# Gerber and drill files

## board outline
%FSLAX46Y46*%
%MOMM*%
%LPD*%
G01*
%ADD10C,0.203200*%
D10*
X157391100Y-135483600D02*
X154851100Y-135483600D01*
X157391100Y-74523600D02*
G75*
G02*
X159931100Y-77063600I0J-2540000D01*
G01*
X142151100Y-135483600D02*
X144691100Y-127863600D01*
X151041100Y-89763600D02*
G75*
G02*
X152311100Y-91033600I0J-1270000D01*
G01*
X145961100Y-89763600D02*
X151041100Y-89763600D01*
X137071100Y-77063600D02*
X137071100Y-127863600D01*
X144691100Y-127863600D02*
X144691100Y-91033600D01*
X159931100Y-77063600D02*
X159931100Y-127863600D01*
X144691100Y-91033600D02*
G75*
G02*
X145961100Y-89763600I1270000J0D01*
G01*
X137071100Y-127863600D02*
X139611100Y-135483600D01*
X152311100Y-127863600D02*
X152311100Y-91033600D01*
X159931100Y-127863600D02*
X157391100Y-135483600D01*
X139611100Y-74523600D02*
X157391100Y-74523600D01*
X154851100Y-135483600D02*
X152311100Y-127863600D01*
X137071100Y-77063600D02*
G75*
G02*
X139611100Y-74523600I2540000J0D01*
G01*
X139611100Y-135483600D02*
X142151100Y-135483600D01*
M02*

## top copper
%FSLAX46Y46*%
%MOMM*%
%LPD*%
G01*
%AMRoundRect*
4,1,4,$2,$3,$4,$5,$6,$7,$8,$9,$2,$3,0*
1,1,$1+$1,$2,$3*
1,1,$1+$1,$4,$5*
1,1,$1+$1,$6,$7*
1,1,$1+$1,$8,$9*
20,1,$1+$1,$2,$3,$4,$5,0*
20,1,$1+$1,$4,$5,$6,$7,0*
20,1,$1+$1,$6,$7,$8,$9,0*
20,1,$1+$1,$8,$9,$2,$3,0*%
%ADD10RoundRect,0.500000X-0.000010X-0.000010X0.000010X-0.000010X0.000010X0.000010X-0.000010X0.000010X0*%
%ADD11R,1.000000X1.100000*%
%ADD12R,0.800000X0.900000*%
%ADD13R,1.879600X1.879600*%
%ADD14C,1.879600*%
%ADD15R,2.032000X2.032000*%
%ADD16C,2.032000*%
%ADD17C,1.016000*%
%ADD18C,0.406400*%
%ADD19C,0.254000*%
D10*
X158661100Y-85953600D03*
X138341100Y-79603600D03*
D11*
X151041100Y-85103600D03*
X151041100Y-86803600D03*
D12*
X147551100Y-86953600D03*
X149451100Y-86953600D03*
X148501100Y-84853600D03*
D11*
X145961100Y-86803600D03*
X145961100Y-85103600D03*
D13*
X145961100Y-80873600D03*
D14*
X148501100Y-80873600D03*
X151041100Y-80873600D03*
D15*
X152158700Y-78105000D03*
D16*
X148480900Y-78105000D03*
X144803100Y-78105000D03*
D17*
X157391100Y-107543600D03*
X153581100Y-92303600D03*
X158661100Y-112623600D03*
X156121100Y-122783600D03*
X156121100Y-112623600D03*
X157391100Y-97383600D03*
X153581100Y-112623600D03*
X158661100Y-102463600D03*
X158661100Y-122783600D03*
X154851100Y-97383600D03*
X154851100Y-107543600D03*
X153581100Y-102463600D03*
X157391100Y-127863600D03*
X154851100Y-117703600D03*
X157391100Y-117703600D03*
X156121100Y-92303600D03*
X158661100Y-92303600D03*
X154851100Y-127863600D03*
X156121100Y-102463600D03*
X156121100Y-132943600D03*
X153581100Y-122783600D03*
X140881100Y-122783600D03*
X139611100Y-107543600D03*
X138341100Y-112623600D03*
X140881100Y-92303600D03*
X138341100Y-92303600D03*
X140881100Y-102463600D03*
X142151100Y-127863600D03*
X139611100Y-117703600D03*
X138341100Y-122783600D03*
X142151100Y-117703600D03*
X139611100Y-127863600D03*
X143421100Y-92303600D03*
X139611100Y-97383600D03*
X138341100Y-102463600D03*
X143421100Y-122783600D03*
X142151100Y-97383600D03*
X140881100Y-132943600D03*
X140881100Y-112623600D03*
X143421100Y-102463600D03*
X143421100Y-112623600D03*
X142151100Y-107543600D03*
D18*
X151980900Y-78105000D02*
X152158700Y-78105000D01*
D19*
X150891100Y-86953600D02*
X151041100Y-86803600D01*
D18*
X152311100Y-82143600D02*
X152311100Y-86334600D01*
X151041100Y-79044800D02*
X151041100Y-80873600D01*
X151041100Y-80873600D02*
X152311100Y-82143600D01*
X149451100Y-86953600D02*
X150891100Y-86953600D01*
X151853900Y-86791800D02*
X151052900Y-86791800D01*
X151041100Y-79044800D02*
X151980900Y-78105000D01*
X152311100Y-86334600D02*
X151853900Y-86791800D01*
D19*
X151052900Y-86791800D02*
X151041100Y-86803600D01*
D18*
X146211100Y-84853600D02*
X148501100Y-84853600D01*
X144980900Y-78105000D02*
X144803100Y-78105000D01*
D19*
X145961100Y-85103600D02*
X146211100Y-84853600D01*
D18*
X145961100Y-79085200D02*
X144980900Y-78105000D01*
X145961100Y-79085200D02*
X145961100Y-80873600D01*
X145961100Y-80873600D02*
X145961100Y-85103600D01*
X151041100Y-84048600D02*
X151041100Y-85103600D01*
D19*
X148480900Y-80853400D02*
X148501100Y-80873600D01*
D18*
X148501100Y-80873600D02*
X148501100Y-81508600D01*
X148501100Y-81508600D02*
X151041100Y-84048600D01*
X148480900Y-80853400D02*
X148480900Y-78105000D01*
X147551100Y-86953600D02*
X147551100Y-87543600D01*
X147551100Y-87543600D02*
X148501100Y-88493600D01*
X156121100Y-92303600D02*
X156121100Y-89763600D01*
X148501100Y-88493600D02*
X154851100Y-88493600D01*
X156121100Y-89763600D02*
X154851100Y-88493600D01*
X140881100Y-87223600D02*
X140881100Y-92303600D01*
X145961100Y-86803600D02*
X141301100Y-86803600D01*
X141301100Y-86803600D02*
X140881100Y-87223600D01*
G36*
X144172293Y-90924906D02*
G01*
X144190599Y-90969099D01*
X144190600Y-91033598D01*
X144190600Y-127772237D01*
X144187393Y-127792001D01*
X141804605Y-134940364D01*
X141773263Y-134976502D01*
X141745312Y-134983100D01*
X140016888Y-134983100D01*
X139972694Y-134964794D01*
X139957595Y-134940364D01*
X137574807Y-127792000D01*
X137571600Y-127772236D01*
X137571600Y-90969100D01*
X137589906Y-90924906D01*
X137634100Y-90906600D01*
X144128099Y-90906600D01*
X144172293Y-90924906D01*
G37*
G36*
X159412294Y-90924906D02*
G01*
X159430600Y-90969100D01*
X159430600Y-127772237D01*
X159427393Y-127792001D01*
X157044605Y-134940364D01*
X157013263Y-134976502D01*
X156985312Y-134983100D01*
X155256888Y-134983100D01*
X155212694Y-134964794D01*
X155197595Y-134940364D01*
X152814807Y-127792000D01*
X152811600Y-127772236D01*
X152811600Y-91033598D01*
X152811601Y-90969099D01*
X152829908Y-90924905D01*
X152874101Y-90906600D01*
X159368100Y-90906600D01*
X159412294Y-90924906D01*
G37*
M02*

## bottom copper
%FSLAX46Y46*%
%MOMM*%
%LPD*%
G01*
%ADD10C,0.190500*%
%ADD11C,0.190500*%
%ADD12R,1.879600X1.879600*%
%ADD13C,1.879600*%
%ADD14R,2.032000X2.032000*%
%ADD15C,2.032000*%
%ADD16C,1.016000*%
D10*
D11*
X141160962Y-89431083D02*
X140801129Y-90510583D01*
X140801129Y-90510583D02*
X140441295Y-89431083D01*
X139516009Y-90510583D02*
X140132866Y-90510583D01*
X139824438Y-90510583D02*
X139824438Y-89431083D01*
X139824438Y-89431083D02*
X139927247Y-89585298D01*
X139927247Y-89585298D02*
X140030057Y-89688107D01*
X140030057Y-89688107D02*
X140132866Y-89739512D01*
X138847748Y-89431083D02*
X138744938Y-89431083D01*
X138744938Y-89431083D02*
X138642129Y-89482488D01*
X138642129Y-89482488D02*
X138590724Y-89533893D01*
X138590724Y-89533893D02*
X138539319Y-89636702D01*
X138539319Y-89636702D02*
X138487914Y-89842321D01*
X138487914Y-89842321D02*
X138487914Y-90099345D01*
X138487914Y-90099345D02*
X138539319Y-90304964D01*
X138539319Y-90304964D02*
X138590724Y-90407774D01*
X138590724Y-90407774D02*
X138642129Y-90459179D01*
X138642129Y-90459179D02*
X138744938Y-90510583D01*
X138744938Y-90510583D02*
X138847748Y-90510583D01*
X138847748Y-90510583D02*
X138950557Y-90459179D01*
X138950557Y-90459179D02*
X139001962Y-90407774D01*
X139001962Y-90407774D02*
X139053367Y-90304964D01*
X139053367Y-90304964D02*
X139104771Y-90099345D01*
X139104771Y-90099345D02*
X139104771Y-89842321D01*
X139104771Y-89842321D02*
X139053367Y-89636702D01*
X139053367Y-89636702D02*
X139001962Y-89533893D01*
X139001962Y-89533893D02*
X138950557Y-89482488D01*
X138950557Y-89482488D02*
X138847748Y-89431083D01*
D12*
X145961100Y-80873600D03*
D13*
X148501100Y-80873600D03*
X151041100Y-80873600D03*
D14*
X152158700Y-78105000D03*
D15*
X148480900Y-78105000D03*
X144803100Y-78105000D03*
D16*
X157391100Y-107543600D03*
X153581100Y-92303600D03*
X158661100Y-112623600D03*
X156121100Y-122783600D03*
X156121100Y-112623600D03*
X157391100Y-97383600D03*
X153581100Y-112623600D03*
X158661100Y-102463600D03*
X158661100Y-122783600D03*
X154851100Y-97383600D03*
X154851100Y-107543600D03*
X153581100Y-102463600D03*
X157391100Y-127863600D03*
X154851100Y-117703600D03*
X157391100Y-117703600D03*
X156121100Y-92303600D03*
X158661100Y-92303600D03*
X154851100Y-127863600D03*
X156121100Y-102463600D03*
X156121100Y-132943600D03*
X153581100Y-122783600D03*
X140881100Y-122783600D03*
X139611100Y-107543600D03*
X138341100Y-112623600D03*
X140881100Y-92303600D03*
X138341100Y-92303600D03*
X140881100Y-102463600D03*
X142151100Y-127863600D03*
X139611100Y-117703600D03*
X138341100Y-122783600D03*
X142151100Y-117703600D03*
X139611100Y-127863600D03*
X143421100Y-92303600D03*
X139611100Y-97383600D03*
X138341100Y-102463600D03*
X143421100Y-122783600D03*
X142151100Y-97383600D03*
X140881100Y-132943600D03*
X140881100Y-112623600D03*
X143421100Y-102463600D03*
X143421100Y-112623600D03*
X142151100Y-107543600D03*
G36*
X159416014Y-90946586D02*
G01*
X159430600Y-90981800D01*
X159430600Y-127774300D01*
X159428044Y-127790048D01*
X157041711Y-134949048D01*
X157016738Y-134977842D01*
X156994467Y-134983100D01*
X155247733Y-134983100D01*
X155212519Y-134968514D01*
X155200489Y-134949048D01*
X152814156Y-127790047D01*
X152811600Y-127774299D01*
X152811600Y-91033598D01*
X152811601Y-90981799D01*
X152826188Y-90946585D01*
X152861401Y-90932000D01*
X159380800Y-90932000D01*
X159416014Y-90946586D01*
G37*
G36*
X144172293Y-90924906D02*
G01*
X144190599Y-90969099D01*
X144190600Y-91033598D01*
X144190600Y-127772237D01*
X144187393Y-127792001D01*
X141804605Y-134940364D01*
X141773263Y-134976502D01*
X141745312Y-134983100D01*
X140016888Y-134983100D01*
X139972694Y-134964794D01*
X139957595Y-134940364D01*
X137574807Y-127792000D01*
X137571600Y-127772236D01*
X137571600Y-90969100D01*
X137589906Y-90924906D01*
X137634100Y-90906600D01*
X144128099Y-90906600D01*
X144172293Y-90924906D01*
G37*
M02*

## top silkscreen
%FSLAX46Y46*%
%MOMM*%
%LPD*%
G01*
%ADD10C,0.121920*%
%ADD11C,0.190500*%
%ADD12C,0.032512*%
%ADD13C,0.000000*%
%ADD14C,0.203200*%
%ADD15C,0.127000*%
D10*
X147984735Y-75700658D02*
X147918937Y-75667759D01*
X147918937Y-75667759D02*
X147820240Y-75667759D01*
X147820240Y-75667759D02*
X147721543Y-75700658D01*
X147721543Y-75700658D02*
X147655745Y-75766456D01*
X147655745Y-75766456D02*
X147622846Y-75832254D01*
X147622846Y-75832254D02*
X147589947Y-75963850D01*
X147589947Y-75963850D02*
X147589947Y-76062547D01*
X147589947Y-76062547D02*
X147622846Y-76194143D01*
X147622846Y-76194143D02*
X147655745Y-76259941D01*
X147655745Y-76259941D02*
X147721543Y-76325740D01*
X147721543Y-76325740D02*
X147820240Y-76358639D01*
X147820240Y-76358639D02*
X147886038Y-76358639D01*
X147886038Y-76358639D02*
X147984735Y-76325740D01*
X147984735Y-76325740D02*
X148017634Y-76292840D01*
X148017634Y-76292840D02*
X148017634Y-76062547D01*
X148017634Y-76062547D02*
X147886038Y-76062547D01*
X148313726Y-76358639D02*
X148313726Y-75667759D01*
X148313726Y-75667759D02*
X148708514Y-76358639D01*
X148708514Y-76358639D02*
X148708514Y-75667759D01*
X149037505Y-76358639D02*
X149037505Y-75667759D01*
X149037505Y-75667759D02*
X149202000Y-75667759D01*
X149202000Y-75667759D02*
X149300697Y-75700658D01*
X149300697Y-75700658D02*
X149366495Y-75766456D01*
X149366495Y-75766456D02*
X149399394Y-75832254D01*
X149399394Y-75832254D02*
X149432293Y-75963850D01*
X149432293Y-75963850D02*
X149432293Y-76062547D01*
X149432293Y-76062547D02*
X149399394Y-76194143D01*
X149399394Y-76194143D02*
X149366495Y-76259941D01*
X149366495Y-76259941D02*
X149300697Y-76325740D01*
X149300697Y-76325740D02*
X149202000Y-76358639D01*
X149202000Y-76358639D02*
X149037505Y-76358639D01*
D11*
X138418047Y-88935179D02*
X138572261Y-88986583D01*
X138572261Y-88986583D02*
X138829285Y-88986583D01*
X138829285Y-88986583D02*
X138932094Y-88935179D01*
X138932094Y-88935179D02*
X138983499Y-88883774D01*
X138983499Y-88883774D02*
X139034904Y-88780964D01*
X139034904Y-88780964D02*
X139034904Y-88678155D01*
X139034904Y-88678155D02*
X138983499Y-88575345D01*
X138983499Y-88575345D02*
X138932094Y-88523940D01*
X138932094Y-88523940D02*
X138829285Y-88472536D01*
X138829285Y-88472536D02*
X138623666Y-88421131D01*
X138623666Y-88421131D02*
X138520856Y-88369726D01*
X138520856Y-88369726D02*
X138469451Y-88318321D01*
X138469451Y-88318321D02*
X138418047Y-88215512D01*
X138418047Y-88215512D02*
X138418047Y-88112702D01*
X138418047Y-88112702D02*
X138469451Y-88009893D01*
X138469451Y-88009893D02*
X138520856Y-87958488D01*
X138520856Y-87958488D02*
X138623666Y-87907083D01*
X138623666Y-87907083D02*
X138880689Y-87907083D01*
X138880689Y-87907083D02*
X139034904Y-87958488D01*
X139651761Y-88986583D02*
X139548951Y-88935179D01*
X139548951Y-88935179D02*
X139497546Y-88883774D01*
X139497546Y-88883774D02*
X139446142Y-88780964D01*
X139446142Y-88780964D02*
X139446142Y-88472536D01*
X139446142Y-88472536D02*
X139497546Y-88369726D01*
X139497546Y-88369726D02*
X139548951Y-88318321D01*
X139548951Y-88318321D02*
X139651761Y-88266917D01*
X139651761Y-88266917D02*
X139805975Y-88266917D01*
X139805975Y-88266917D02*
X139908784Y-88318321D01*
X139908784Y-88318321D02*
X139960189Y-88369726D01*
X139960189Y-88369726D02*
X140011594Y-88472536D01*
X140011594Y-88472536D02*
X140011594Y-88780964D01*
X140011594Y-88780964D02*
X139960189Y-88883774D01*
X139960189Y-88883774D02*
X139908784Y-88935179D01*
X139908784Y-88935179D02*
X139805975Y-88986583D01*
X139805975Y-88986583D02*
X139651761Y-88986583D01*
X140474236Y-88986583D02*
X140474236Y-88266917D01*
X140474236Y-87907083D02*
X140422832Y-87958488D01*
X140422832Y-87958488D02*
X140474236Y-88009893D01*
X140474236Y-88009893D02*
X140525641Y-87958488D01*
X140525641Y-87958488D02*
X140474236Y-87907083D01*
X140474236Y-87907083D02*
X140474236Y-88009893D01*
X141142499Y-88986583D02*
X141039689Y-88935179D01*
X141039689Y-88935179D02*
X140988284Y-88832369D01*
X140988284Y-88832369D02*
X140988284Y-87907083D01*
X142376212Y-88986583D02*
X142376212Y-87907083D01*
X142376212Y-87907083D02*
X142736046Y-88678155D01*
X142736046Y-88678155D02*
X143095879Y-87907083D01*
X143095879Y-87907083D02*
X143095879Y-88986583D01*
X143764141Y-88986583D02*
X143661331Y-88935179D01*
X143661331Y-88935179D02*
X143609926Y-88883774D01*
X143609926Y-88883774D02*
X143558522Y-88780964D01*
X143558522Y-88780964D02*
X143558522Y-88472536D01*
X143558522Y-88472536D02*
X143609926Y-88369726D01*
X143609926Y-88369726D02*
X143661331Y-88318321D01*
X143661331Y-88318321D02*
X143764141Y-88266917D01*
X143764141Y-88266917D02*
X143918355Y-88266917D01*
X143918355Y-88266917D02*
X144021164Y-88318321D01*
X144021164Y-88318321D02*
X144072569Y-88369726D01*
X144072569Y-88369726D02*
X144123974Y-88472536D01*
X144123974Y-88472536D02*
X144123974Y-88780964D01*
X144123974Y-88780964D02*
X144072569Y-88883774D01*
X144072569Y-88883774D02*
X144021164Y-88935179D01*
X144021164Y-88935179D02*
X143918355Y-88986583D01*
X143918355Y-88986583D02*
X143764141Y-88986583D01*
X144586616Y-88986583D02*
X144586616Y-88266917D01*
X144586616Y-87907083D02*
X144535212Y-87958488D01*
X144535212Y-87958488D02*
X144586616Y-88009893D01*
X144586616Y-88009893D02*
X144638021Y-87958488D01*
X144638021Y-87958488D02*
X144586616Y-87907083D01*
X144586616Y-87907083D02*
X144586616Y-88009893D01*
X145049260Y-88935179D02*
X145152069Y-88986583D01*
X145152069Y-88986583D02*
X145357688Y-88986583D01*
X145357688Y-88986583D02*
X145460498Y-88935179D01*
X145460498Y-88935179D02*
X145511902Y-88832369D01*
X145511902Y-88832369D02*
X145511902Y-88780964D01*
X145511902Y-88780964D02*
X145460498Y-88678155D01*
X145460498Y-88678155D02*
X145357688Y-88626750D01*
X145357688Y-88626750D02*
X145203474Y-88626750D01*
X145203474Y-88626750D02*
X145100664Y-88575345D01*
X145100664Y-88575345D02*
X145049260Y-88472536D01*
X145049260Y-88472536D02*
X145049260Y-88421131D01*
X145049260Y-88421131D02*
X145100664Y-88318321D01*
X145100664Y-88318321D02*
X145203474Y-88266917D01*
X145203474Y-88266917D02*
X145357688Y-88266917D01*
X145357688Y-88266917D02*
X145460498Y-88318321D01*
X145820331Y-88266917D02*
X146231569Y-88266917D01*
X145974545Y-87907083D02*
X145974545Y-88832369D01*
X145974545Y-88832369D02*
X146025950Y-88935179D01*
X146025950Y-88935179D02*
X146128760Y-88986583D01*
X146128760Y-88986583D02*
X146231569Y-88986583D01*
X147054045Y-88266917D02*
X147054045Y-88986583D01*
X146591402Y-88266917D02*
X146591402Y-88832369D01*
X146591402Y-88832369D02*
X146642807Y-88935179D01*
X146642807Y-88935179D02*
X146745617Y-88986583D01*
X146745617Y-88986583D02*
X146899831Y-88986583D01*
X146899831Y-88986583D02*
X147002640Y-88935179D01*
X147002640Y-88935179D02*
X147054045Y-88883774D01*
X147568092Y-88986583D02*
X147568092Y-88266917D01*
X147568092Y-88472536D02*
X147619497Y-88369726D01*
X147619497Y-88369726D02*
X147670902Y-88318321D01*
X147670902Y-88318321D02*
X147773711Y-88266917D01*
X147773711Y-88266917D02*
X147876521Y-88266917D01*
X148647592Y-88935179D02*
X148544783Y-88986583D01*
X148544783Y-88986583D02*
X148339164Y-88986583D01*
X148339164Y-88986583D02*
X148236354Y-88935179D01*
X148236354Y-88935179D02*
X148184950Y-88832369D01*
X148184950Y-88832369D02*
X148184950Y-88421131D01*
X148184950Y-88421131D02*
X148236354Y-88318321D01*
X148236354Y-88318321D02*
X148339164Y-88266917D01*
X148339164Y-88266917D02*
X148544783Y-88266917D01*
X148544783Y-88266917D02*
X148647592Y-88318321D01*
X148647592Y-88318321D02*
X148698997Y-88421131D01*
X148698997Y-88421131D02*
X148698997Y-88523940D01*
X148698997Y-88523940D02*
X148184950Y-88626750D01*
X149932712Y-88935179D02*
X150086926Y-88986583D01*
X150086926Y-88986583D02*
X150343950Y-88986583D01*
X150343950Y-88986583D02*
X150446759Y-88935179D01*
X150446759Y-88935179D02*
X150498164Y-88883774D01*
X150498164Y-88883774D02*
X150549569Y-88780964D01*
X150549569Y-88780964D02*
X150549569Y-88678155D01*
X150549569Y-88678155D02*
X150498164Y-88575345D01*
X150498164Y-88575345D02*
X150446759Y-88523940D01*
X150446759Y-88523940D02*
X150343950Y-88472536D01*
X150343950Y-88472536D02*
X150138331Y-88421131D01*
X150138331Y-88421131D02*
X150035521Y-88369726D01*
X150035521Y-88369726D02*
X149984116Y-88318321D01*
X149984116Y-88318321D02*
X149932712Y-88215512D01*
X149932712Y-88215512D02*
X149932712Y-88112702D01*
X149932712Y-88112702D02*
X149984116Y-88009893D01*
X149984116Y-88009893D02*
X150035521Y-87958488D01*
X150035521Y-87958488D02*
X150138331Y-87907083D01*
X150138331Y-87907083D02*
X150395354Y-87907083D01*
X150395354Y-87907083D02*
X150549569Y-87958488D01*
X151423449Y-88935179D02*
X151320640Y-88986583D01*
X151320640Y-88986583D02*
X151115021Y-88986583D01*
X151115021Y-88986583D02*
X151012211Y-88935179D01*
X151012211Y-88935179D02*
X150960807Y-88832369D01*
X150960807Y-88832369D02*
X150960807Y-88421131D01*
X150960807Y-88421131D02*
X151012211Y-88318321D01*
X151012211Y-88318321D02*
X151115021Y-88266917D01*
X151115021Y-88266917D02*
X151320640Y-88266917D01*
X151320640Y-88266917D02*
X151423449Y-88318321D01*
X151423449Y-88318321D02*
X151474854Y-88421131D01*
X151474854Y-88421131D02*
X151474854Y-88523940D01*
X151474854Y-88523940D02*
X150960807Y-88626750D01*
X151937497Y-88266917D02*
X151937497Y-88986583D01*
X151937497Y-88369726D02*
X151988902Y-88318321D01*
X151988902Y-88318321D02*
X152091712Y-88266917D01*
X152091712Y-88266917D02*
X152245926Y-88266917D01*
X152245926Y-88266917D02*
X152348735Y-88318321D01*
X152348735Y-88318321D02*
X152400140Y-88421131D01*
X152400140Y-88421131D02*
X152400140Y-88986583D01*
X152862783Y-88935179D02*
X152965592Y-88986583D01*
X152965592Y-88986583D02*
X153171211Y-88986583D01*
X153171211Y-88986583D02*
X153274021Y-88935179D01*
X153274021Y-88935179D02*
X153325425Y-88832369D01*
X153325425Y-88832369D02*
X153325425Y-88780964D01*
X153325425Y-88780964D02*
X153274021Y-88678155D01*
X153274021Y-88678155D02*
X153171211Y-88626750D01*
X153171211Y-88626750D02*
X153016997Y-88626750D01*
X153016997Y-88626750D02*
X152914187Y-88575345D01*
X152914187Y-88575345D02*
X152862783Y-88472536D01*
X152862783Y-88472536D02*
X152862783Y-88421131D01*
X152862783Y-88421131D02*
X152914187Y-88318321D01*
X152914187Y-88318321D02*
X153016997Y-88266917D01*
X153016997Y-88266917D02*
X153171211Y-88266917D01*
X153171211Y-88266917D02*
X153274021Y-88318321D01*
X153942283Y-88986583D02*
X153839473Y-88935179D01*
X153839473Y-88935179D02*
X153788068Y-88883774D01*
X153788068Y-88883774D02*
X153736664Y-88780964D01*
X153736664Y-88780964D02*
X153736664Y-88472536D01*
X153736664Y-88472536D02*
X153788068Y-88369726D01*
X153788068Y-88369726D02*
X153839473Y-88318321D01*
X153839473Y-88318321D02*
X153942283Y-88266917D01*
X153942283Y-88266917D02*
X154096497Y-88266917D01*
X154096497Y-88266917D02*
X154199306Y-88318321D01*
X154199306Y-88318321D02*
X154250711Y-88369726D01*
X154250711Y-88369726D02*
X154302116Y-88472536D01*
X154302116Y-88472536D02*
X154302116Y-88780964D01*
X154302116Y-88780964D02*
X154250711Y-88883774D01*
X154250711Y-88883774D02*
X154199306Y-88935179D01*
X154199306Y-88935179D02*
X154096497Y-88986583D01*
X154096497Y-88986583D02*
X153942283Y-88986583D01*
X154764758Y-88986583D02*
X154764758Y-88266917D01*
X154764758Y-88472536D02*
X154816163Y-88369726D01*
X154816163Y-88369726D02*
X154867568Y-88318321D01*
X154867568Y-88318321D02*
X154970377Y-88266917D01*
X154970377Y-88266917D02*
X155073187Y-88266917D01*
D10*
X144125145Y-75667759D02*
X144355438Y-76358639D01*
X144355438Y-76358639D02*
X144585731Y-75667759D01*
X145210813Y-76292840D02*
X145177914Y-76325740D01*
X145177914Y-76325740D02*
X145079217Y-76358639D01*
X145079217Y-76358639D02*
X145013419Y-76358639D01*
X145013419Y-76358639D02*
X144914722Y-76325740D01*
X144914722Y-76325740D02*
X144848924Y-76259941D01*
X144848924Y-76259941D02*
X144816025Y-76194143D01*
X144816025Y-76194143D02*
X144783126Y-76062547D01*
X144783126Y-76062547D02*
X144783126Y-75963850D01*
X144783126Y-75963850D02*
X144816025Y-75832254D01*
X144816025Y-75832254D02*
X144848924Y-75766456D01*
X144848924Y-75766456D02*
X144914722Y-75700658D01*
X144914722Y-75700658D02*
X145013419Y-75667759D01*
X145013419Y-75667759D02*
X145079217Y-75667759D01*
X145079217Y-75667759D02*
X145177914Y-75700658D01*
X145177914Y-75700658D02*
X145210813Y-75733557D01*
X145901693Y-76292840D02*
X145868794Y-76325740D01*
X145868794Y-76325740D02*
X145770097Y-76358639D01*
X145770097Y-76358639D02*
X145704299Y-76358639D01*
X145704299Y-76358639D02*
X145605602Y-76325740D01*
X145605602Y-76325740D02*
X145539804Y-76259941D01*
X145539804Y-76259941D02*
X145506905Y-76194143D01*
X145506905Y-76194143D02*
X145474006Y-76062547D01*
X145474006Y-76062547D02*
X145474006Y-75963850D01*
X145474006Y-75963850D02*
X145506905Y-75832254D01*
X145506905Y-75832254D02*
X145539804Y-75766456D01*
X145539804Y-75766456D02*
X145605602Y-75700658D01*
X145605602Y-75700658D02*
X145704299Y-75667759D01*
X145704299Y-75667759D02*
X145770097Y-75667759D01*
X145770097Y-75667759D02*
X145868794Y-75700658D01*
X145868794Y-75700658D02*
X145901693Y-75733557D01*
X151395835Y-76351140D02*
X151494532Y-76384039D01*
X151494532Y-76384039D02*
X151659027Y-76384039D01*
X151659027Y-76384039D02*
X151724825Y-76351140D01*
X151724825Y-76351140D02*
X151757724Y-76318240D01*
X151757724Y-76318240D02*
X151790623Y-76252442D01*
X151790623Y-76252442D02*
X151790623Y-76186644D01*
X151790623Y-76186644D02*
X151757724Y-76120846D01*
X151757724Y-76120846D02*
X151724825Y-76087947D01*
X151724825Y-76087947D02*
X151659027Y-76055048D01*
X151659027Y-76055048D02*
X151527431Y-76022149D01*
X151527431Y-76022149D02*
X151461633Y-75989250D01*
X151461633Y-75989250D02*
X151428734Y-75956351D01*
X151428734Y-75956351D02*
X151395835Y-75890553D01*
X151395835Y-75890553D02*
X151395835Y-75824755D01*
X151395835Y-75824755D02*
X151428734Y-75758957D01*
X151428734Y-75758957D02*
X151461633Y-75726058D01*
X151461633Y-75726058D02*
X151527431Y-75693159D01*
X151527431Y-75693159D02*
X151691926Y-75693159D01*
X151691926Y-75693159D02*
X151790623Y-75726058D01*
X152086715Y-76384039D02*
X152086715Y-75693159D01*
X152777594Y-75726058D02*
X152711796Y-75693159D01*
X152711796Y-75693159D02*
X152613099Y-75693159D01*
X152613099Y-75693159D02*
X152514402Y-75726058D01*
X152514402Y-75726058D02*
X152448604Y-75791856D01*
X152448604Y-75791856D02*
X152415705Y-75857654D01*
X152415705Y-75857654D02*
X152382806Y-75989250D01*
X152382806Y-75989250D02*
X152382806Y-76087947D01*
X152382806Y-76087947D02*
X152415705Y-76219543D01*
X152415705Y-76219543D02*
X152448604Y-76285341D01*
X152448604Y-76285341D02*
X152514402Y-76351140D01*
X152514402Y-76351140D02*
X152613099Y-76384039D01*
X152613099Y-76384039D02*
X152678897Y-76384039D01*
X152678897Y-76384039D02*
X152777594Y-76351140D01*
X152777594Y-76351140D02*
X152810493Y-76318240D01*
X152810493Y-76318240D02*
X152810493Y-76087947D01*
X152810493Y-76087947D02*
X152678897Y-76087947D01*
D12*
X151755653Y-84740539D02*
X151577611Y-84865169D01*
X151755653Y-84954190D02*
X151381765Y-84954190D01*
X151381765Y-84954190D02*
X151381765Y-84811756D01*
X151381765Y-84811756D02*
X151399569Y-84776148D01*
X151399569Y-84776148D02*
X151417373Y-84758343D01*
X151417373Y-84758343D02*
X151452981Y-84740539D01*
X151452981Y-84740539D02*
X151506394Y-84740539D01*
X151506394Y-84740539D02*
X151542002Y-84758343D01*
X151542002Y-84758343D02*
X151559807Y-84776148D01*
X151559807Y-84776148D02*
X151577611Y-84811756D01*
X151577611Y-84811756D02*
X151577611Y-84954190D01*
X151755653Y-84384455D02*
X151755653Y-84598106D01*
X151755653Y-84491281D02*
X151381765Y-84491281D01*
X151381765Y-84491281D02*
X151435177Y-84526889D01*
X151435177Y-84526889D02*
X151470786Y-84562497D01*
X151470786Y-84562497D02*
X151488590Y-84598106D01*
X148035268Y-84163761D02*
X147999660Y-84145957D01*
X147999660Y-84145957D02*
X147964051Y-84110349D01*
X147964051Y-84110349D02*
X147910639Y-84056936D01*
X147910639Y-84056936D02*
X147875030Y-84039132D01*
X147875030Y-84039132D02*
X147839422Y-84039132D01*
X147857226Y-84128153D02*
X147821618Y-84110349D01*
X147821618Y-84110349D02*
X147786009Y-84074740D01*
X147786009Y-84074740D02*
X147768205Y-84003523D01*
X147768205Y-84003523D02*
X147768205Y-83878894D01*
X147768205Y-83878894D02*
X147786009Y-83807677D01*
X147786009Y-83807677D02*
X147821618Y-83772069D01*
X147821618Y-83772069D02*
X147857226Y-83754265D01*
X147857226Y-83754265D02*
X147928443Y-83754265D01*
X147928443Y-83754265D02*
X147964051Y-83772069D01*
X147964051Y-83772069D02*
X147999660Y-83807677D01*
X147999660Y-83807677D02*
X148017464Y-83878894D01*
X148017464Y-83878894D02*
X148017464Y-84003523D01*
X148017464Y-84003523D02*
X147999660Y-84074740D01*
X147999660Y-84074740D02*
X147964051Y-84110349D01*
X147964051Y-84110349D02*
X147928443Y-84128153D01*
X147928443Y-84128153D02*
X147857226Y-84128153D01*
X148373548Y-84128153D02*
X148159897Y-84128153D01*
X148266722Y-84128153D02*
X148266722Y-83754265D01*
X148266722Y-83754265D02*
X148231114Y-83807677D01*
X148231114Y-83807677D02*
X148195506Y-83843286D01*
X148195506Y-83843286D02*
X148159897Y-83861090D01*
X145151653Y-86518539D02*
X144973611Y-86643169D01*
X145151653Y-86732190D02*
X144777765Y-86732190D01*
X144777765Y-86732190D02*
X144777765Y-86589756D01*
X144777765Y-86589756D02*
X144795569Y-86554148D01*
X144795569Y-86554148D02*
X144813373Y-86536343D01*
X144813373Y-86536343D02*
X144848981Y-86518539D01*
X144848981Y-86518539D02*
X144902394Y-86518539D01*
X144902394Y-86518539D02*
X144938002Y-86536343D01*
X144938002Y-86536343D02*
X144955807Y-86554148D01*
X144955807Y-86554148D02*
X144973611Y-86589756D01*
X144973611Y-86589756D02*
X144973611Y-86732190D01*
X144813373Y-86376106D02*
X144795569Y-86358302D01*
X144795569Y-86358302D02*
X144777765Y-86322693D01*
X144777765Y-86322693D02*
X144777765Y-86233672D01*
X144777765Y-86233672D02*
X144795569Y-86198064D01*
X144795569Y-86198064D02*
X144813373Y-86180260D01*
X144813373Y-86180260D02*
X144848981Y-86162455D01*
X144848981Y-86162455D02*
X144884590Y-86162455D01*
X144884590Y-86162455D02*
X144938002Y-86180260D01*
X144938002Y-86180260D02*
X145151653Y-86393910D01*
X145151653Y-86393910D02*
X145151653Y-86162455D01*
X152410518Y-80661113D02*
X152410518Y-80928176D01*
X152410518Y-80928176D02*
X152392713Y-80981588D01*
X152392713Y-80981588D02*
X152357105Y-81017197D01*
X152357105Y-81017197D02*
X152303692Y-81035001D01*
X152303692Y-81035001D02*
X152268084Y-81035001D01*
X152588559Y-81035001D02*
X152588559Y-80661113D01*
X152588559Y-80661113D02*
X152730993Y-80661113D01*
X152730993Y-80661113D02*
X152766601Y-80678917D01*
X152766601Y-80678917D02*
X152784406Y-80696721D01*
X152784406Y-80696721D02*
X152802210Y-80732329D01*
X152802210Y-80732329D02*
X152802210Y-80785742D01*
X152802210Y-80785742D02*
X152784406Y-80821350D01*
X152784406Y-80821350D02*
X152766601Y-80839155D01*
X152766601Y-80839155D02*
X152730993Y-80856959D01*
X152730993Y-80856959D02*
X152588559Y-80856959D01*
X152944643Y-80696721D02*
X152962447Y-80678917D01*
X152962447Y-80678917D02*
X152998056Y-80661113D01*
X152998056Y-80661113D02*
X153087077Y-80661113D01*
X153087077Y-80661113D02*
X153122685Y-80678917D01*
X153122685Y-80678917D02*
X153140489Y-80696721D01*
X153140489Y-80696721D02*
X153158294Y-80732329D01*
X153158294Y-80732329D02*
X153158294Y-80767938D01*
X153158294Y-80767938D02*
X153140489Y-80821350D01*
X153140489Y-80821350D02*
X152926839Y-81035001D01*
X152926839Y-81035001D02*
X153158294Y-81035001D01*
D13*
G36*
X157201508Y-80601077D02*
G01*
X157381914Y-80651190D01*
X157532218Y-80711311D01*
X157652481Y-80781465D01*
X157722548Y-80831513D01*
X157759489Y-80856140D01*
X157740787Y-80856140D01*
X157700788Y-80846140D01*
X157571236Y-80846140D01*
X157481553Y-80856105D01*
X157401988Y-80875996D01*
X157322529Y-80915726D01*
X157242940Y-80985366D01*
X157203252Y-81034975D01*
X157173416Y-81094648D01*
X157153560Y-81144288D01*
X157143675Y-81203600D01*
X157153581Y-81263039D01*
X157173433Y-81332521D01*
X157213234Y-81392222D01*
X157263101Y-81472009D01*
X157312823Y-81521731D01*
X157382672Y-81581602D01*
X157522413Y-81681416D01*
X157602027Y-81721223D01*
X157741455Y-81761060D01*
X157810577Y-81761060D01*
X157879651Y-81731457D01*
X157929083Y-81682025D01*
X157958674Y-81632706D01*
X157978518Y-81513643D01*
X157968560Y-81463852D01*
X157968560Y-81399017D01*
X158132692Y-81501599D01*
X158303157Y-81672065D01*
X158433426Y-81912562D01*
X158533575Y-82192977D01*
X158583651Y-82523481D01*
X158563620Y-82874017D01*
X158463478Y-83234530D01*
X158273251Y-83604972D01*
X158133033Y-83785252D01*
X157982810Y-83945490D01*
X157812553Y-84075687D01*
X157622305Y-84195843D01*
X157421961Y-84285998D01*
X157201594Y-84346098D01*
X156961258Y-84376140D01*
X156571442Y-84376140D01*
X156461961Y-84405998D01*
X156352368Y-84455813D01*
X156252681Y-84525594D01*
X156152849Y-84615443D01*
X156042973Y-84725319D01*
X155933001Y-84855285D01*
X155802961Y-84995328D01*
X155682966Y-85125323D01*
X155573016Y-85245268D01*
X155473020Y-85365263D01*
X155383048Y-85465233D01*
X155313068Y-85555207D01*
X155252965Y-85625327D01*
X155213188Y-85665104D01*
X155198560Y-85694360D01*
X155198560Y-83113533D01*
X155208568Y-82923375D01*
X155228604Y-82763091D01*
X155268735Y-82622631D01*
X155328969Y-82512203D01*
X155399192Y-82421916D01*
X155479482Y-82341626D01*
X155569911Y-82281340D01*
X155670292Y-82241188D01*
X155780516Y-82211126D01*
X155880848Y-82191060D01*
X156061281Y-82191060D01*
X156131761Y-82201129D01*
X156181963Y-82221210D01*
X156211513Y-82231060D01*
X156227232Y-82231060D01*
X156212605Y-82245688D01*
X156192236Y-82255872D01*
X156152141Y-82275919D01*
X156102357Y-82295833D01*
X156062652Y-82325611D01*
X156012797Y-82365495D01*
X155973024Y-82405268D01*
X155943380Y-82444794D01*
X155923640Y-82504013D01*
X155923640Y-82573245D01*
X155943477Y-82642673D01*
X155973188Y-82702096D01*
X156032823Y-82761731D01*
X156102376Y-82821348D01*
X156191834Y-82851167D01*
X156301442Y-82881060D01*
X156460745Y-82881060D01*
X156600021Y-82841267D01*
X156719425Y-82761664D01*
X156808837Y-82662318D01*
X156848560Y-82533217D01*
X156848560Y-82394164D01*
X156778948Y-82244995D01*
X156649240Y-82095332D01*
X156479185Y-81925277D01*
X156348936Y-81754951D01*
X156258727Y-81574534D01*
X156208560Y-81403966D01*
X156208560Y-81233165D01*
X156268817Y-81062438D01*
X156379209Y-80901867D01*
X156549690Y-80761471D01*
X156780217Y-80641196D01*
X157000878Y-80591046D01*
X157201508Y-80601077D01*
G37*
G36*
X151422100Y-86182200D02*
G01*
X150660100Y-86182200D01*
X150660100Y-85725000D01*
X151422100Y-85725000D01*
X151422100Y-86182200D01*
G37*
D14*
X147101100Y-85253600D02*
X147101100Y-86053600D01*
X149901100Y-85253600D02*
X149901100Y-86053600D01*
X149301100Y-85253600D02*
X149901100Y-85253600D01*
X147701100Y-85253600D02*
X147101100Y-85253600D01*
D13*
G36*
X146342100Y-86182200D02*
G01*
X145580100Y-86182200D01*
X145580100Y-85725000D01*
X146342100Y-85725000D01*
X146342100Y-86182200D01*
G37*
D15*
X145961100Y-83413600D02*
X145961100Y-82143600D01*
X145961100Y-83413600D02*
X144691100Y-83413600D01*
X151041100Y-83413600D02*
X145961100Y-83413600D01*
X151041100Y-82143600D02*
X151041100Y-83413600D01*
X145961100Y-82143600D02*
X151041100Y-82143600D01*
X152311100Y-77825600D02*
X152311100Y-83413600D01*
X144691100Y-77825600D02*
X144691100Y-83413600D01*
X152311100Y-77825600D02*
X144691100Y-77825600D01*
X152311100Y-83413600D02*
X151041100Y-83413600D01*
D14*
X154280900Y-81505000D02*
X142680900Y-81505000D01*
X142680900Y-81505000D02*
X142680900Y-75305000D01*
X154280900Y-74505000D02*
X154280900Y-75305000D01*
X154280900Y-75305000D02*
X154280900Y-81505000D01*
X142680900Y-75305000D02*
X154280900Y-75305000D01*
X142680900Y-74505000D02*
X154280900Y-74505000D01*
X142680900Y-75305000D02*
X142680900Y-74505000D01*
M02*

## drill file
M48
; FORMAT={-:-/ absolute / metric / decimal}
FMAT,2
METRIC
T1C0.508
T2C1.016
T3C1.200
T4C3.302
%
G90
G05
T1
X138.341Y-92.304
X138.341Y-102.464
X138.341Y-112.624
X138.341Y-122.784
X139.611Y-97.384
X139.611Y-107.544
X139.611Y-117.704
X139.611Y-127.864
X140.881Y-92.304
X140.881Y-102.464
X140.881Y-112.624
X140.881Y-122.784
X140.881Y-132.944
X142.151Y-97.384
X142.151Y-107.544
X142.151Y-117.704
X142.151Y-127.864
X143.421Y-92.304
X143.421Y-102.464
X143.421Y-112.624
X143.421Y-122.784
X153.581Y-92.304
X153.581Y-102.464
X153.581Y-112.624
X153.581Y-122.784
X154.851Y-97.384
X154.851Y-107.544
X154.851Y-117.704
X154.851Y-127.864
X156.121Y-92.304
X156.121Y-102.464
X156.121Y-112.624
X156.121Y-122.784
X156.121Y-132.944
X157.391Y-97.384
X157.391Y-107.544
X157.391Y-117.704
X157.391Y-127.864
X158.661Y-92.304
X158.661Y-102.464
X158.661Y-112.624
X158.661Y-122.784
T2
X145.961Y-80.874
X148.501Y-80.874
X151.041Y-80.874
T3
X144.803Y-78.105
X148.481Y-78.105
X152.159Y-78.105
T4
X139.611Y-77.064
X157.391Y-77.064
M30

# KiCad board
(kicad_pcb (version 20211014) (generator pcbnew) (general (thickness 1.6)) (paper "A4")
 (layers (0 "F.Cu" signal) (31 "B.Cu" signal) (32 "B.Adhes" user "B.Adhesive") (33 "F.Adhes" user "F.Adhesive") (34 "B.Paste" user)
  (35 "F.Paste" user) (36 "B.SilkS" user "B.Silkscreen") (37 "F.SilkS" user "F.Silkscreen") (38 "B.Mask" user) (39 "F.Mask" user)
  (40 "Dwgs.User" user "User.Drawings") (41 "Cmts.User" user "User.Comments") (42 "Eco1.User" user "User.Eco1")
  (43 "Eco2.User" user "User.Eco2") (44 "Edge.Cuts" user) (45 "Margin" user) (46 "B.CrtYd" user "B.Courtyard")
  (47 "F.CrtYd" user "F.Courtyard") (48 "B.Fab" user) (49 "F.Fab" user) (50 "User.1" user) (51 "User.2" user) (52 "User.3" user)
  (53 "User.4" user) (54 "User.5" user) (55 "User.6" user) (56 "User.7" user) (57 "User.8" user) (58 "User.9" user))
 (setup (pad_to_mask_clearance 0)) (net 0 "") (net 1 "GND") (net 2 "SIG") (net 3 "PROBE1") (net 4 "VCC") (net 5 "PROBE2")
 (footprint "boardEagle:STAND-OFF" (layer "F.Cu") (at 157.3911 77.0636)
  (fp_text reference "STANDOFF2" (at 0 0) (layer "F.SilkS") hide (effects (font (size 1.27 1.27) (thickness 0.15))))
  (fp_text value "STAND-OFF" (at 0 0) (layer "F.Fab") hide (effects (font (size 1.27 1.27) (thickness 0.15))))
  (pad "" np_thru_hole circle (at 0 0) (size 3.302 3.302) (drill 3.302) (layers *.Cu *.Mask)))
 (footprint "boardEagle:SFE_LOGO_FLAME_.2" (layer "F.Cu") (at 154.8511 85.9536)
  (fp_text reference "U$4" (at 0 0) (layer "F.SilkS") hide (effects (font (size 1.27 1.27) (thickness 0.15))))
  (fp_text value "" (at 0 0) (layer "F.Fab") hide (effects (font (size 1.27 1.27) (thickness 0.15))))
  (fp_poly
   (pts (xy 2.350408 -5.352523) (xy 2.530814 -5.30241) (xy 2.681118 -5.242289) (xy 2.801381 -5.172135) (xy 2.871448 -5.122087)
    (xy 2.908389 -5.09746) (xy 2.889687 -5.09746) (xy 2.849688 -5.10746) (xy 2.720136 -5.10746) (xy 2.630453 -5.097495)
    (xy 2.550888 -5.077604) (xy 2.471429 -5.037874) (xy 2.39184 -4.968234) (xy 2.352152 -4.918625) (xy 2.322316 -4.858952)
    (xy 2.30246 -4.809312) (xy 2.292575 -4.75) (xy 2.302481 -4.690561) (xy 2.322333 -4.621079) (xy 2.362134 -4.561378)
    (xy 2.412001 -4.481591) (xy 2.461723 -4.431869) (xy 2.531572 -4.371998) (xy 2.671313 -4.272184) (xy 2.750927 -4.232377)
    (xy 2.890355 -4.19254) (xy 2.959477 -4.19254) (xy 3.028551 -4.222143) (xy 3.077983 -4.271575) (xy 3.107574 -4.320894)
    (xy 3.127418 -4.439957) (xy 3.11746 -4.489748) (xy 3.11746 -4.554583) (xy 3.281592 -4.452001) (xy 3.452057 -4.281535)
    (xy 3.582326 -4.041038) (xy 3.682475 -3.760623) (xy 3.732551 -3.430119) (xy 3.71252 -3.079583) (xy 3.612378 -2.71907)
    (xy 3.422151 -2.348628) (xy 3.281933 -2.168348) (xy 3.13171 -2.00811) (xy 2.961453 -1.877913) (xy 2.771205 -1.757757)
    (xy 2.570861 -1.667602) (xy 2.350494 -1.607502) (xy 2.110158 -1.57746) (xy 1.720342 -1.57746) (xy 1.610861 -1.547602)
    (xy 1.501268 -1.497787) (xy 1.401581 -1.428006) (xy 1.301749 -1.338157) (xy 1.191873 -1.228281) (xy 1.081901 -1.098315)
    (xy 0.951861 -0.958272) (xy 0.831866 -0.828277) (xy 0.721916 -0.708332) (xy 0.62192 -0.588337) (xy 0.531948 -0.488367)
    (xy 0.461968 -0.398393) (xy 0.401865 -0.328273) (xy 0.362088 -0.288496) (xy 0.34746 -0.25924) (xy 0.34746 -2.840067)
    (xy 0.357468 -3.030225) (xy 0.377504 -3.190509) (xy 0.417635 -3.330969) (xy 0.477869 -3.441397) (xy 0.548092 -3.531684)
    (xy 0.628382 -3.611974) (xy 0.718811 -3.67226) (xy 0.819192 -3.712412) (xy 0.929416 -3.742474) (xy 1.029748 -3.76254)
    (xy 1.210181 -3.76254) (xy 1.280661 -3.752471) (xy 1.330863 -3.73239) (xy 1.360413 -3.72254) (xy 1.376132 -3.72254)
    (xy 1.361505 -3.707912) (xy 1.341136 -3.697728) (xy 1.301041 -3.677681) (xy 1.251257 -3.657767) (xy 1.211552 -3.627989)
    (xy 1.161697 -3.588105) (xy 1.121924 -3.548332) (xy 1.09228 -3.508806) (xy 1.07254 -3.449587) (xy 1.07254 -3.380355)
    (xy 1.092377 -3.310927) (xy 1.122088 -3.251504) (xy 1.181723 -3.191869) (xy 1.251276 -3.132252) (xy 1.340734 -3.102433)
    (xy 1.450342 -3.07254) (xy 1.609645 -3.07254) (xy 1.748921 -3.112333) (xy 1.868325 -3.191936) (xy 1.957737 -3.291282)
    (xy 1.99746 -3.420383) (xy 1.99746 -3.559436) (xy 1.927848 -3.708605) (xy 1.79814 -3.858268) (xy 1.628085 -4.028323)
    (xy 1.497836 -4.198649) (xy 1.407627 -4.379066) (xy 1.35746 -4.549634) (xy 1.35746 -4.720435) (xy 1.417717 -4.891162)
    (xy 1.528109 -5.051733) (xy 1.69859 -5.192129) (xy 1.929117 -5.312404) (xy 2.149778 -5.362554))
   (layer "F.SilkS") (width 0) (fill solid)))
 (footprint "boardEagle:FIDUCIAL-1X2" (layer "F.Cu") (at 158.6611 85.9536)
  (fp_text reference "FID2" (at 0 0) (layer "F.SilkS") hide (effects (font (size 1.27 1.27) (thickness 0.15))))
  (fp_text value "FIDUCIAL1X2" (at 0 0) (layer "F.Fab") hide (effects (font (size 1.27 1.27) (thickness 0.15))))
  (pad "1" smd roundrect (at 0 0) (size 1 1) (layers "F.Cu" "F.Mask") (roundrect_rratio 0.5) (solder_mask_margin 0.1016)))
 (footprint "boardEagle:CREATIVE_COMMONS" (layer "F.Cu") (at 129.4511 145.6436)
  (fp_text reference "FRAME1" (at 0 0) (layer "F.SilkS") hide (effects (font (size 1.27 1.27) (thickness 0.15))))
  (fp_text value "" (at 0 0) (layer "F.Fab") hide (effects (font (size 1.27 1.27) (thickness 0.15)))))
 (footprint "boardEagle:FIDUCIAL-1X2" (layer "F.Cu") (at 138.3411 79.6036)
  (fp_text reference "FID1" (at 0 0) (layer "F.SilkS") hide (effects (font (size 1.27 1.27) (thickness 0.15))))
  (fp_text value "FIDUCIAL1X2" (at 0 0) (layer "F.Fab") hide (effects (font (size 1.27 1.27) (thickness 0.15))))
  (pad "1" smd roundrect (at 0 0) (size 1 1) (layers "F.Cu" "F.Mask") (roundrect_rratio 0.5) (solder_mask_margin 0.1016)))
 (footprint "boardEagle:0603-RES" (layer "F.Cu") (at 151.0411 85.9536 -90)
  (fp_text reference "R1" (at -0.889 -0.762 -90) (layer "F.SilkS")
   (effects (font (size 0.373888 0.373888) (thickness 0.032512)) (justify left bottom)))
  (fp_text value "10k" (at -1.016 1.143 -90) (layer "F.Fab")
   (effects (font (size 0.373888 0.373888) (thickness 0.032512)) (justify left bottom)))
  (fp_poly (pts (xy -0.2286 0.381) (xy 0.2286 0.381) (xy 0.2286 -0.381) (xy -0.2286 -0.381)) (layer "F.SilkS") (width 0) (fill solid))
  (pad "1" smd rect (at -0.85 0 270) (size 1.1 1) (layers "F.Cu" "F.Paste" "F.Mask") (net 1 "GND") (solder_mask_margin 0.1016))
  (pad "2" smd rect (at 0.85 0 270) (size 1.1 1) (layers "F.Cu" "F.Paste" "F.Mask") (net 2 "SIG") (solder_mask_margin 0.1016)))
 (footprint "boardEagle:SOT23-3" (layer "F.Cu") (at 148.5011 85.9536)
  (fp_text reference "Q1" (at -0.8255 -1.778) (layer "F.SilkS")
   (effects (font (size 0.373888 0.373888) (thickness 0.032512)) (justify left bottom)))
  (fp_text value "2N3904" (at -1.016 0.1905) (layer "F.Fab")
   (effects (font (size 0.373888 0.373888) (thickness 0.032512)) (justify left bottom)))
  (fp_line (start -1.4 -0.7) (end -1.4 0.1) (layer "F.SilkS") (width 0.2032))
  (fp_line (start 1.4 -0.7) (end 1.4 0.1) (layer "F.SilkS") (width 0.2032))
  (fp_line (start 0.8 -0.7) (end 1.4 -0.7) (layer "F.SilkS") (width 0.2032))
  (fp_line (start -0.8 -0.7) (end -1.4 -0.7) (layer "F.SilkS") (width 0.2032))
  (pad "1" smd rect (at -0.95 1) (size 0.8 0.9) (layers "F.Cu" "F.Paste" "F.Mask") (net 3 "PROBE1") (solder_mask_margin 0.1016))
  (pad "2" smd rect (at 0.95 1) (size 0.8 0.9) (layers "F.Cu" "F.Paste" "F.Mask") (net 2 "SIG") (solder_mask_margin 0.1016))
  (pad "3" smd rect (at 0 -1.1) (size 0.8 0.9) (layers "F.Cu" "F.Paste" "F.Mask") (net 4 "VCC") (solder_mask_margin 0.1016)))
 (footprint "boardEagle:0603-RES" (layer "F.Cu") (at 145.9611 85.9536 90)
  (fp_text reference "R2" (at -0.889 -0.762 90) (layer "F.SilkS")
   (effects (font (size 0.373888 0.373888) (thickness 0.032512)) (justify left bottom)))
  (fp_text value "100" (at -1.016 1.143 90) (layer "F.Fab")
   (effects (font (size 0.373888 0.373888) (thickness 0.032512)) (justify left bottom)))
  (fp_poly (pts (xy -0.2286 0.381) (xy 0.2286 0.381) (xy 0.2286 -0.381) (xy -0.2286 -0.381)) (layer "F.SilkS") (width 0) (fill solid))
  (pad "1" smd rect (at -0.85 0 90) (size 1.1 1) (layers "F.Cu" "F.Paste" "F.Mask") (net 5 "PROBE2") (solder_mask_margin 0.1016))
  (pad "2" smd rect (at 0.85 0 90) (size 1.1 1) (layers "F.Cu" "F.Paste" "F.Mask") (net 4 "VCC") (solder_mask_margin 0.1016)))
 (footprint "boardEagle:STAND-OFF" (layer "F.Cu") (at 139.6111 77.0636)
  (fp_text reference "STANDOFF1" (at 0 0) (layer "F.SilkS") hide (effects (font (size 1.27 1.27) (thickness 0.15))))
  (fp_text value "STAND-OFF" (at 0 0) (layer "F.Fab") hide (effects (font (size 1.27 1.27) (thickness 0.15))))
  (pad "" np_thru_hole circle (at 0 0) (size 3.302 3.302) (drill 3.302) (layers *.Cu *.Mask)))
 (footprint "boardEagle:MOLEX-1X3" (layer "F.Cu") (at 145.9611 80.8736)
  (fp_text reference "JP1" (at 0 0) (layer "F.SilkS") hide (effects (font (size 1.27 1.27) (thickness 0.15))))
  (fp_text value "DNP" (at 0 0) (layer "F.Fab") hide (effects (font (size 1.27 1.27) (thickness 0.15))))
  (fp_line (start 0 2.54) (end 0 1.27) (layer "F.SilkS") (width 0.127))
  (fp_line (start 0 2.54) (end -1.27 2.54) (layer "F.SilkS") (width 0.127))
  (fp_line (start 5.08 2.54) (end 0 2.54) (layer "F.SilkS") (width 0.127))
  (fp_line (start 5.08 1.27) (end 5.08 2.54) (layer "F.SilkS") (width 0.127))
  (fp_line (start 0 1.27) (end 5.08 1.27) (layer "F.SilkS") (width 0.127))
  (fp_line (start 6.35 -3.048) (end 6.35 2.54) (layer "F.SilkS") (width 0.127))
  (fp_line (start -1.27 -3.048) (end -1.27 2.54) (layer "F.SilkS") (width 0.127))
  (fp_line (start 6.35 -3.048) (end -1.27 -3.048) (layer "F.SilkS") (width 0.127))
  (fp_line (start 6.35 2.54) (end 5.08 2.54) (layer "F.SilkS") (width 0.127))
  (pad "1" thru_hole rect (at 0 0) (size 1.8796 1.8796) (drill 1.016) (layers *.Cu *.Mask) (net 4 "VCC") (solder_mask_margin 0.1016))
  (pad "2" thru_hole circle (at 2.54 0) (size 1.8796 1.8796) (drill 1.016) (layers *.Cu *.Mask) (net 1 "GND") (solder_mask_margin 0.1016))
  (pad "3" thru_hole circle (at 5.08 0) (size 1.8796 1.8796) (drill 1.016) (layers *.Cu *.Mask) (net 2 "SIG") (solder_mask_margin 0.1016)))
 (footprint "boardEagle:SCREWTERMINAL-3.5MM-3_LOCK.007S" (layer "F.Cu") (at 151.9809 78.105 180)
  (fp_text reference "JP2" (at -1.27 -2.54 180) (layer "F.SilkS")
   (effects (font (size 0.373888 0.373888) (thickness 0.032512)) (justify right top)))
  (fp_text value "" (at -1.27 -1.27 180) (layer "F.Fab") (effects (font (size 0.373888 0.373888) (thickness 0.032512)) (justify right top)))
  (fp_line (start -2.3 -3.4) (end 9.3 -3.4) (layer "F.SilkS") (width 0.2032))
  (fp_line (start 9.3 -3.4) (end 9.3 2.8) (layer "F.SilkS") (width 0.2032))
  (fp_line (start -2.3 3.6) (end -2.3 2.8) (layer "F.SilkS") (width 0.2032))
  (fp_line (start -2.3 2.8) (end -2.3 -3.4) (layer "F.SilkS") (width 0.2032))
  (fp_line (start 9.3 2.8) (end -2.3 2.8) (layer "F.SilkS") (width 0.2032))
  (fp_line (start 9.3 3.6) (end -2.3 3.6) (layer "F.SilkS") (width 0.2032))
  (fp_line (start 9.3 2.8) (end 9.3 3.6) (layer "F.SilkS") (width 0.2032))
  (pad "1" thru_hole rect (at -0.1778 0 180) (size 2.032 2.032) (drill 1.2) (layers *.Cu *.Mask) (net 2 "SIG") (solder_mask_margin 0.1016))
  (pad "2" thru_hole circle (at 3.5 0 180) (size 2.032 2.032) (drill 1.2) (layers *.Cu *.Mask) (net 1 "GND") (solder_mask_margin 0.1016))
  (pad "3" thru_hole circle (at 7.1778 0 180) (size 2.032 2.032) (drill 1.2) (layers *.Cu *.Mask) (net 4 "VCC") (solder_mask_margin 0.1016)))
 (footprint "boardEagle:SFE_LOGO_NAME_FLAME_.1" (layer "B.Cu") (at 154.8511 87.2236 180)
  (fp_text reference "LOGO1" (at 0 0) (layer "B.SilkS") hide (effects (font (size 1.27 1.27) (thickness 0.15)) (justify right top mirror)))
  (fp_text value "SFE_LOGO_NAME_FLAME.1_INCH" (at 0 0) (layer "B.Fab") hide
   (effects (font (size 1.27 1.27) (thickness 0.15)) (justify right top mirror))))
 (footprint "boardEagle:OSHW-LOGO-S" (layer "B.Cu") (at 157.3911 80.8736 180)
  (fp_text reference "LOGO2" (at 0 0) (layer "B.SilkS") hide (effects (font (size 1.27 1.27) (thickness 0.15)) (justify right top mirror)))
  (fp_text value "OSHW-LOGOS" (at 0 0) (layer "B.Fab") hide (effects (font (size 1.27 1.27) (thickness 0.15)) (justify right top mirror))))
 (gr_line (start 157.3911 135.4836) (end 154.8511 135.4836) (layer "Edge.Cuts") (width 0.2032))
 (gr_arc (start 157.3911 74.5236) (mid 159.187151 75.267549) (end 159.9311 77.0636) (layer "Edge.Cuts") (width 0.2032))
 (gr_line (start 142.1511 135.4836) (end 144.6911 127.8636) (layer "Edge.Cuts") (width 0.2032))
 (gr_arc (start 151.0411 89.7636) (mid 151.939126 90.135574) (end 152.3111 91.0336) (layer "Edge.Cuts") (width 0.2032))
 (gr_line (start 145.9611 89.7636) (end 151.0411 89.7636) (layer "Edge.Cuts") (width 0.2032))
 (gr_line (start 137.0711 77.0636) (end 137.0711 127.8636) (layer "Edge.Cuts") (width 0.2032))
 (gr_line (start 144.6911 127.8636) (end 144.6911 91.0336) (layer "Edge.Cuts") (width 0.2032))
 (gr_line (start 159.9311 77.0636) (end 159.9311 127.8636) (layer "Edge.Cuts") (width 0.2032))
 (gr_arc (start 144.6911 91.0336) (mid 145.063074 90.135574) (end 145.9611 89.7636) (layer "Edge.Cuts") (width 0.2032))
 (gr_line (start 137.0711 127.8636) (end 139.6111 135.4836) (layer "Edge.Cuts") (width 0.2032))
 (gr_line (start 152.3111 127.8636) (end 152.3111 91.0336) (layer "Edge.Cuts") (width 0.2032))
 (gr_line (start 159.9311 127.8636) (end 157.3911 135.4836) (layer "Edge.Cuts") (width 0.2032))
 (gr_line (start 139.6111 74.5236) (end 157.3911 74.5236) (layer "Edge.Cuts") (width 0.2032))
 (gr_line (start 154.8511 135.4836) (end 152.3111 127.8636) (layer "Edge.Cuts") (width 0.2032))
 (gr_arc (start 137.0711 77.0636) (mid 137.815049 75.267549) (end 139.6111 74.5236) (layer "Edge.Cuts") (width 0.2032))
 (gr_line (start 139.6111 135.4836) (end 142.1511 135.4836) (layer "Edge.Cuts") (width 0.2032))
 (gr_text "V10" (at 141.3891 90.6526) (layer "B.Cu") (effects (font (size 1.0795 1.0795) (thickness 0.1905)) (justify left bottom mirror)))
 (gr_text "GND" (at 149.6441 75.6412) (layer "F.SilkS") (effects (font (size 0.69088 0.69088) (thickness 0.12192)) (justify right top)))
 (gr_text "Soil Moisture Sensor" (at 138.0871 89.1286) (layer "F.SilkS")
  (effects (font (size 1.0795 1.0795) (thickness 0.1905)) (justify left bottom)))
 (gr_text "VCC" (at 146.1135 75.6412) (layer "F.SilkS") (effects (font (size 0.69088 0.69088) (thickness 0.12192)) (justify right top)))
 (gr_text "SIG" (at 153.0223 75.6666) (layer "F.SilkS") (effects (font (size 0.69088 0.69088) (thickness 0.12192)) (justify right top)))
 (segment (start 151.9809 78.105) (end 152.1587 78.105) (width 0.4064) (layer "F.Cu") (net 2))
 (segment (start 150.8911 86.9536) (end 151.0411 86.8036) (width 0.254) (layer "F.Cu") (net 2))
 (segment (start 152.3111 82.1436) (end 152.3111 86.3346) (width 0.4064) (layer "F.Cu") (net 2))
 (segment (start 151.0411 79.0448) (end 151.0411 80.8736) (width 0.4064) (layer "F.Cu") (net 2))
 (segment (start 151.0411 80.8736) (end 152.3111 82.1436) (width 0.4064) (layer "F.Cu") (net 2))
 (segment (start 149.4511 86.9536) (end 150.8911 86.9536) (width 0.4064) (layer "F.Cu") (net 2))
 (segment (start 151.8539 86.7918) (end 151.0529 86.7918) (width 0.4064) (layer "F.Cu") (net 2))
 (segment (start 151.0411 79.0448) (end 151.9809 78.105) (width 0.4064) (layer "F.Cu") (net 2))
 (segment (start 152.3111 86.3346) (end 151.8539 86.7918) (width 0.4064) (layer "F.Cu") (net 2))
 (segment (start 151.0529 86.7918) (end 151.0411 86.8036) (width 0.254) (layer "F.Cu") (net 2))
 (segment (start 146.2111 84.8536) (end 148.5011 84.8536) (width 0.4064) (layer "F.Cu") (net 4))
 (segment (start 144.9809 78.105) (end 144.8031 78.105) (width 0.4064) (layer "F.Cu") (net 4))
 (segment (start 145.9611 85.1036) (end 146.2111 84.8536) (width 0.254) (layer "F.Cu") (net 4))
 (segment (start 145.9611 79.0852) (end 144.9809 78.105) (width 0.4064) (layer "F.Cu") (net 4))
 (segment (start 145.9611 79.0852) (end 145.9611 80.8736) (width 0.4064) (layer "F.Cu") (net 4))
 (segment (start 145.9611 80.8736) (end 145.9611 85.1036) (width 0.4064) (layer "F.Cu") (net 4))
 (segment (start 151.0411 84.0486) (end 151.0411 85.1036) (width 0.4064) (layer "F.Cu") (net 1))
 (segment (start 148.4809 80.8534) (end 148.5011 80.8736) (width 0.254) (layer "F.Cu") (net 1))
 (segment (start 148.5011 80.8736) (end 148.5011 81.5086) (width 0.4064) (layer "F.Cu") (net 1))
 (segment (start 148.5011 81.5086) (end 151.0411 84.0486) (width 0.4064) (layer "F.Cu") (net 1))
 (segment (start 148.4809 80.8534) (end 148.4809 78.105) (width 0.4064) (layer "F.Cu") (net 1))
 (segment (start 147.5511 86.9536) (end 147.5511 87.5436) (width 0.4064) (layer "F.Cu") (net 3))
 (segment (start 147.5511 87.5436) (end 148.5011 88.4936) (width 0.4064) (layer "F.Cu") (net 3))
 (segment (start 156.1211 92.3036) (end 156.1211 89.7636) (width 0.4064) (layer "F.Cu") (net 3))
 (segment (start 148.5011 88.4936) (end 154.8511 88.4936) (width 0.4064) (layer "F.Cu") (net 3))
 (segment (start 156.1211 89.7636) (end 154.8511 88.4936) (width 0.4064) (layer "F.Cu") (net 3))
 (via (at 157.3911 107.5436) (size 1.016) (drill 0.508) (layers "F.Cu" "B.Cu") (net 3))
 (via (at 153.5811 92.3036) (size 1.016) (drill 0.508) (layers "F.Cu" "B.Cu") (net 3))
 (via (at 158.6611 112.6236) (size 1.016) (drill 0.508) (layers "F.Cu" "B.Cu") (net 3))
 (via (at 156.1211 122.7836) (size 1.016) (drill 0.508) (layers "F.Cu" "B.Cu") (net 3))
 (via (at 156.1211 112.6236) (size 1.016) (drill 0.508) (layers "F.Cu" "B.Cu") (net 3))
 (via (at 157.3911 97.3836) (size 1.016) (drill 0.508) (layers "F.Cu" "B.Cu") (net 3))
 (via (at 153.5811 112.6236) (size 1.016) (drill 0.508) (layers "F.Cu" "B.Cu") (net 3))
 (via (at 158.6611 102.4636) (size 1.016) (drill 0.508) (layers "F.Cu" "B.Cu") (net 3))
 (via (at 158.6611 122.7836) (size 1.016) (drill 0.508) (layers "F.Cu" "B.Cu") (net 3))
 (via (at 154.8511 97.3836) (size 1.016) (drill 0.508) (layers "F.Cu" "B.Cu") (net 3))
 (via (at 154.8511 107.5436) (size 1.016) (drill 0.508) (layers "F.Cu" "B.Cu") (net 3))
 (via (at 153.5811 102.4636) (size 1.016) (drill 0.508) (layers "F.Cu" "B.Cu") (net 3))
 (via (at 157.3911 127.8636) (size 1.016) (drill 0.508) (layers "F.Cu" "B.Cu") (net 3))
 (via (at 154.8511 117.7036) (size 1.016) (drill 0.508) (layers "F.Cu" "B.Cu") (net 3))
 (via (at 157.3911 117.7036) (size 1.016) (drill 0.508) (layers "F.Cu" "B.Cu") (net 3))
 (via (at 156.1211 92.3036) (size 1.016) (drill 0.508) (layers "F.Cu" "B.Cu") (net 3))
 (via (at 158.6611 92.3036) (size 1.016) (drill 0.508) (layers "F.Cu" "B.Cu") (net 3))
 (via (at 154.8511 127.8636) (size 1.016) (drill 0.508) (layers "F.Cu" "B.Cu") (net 3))
 (via (at 156.1211 102.4636) (size 1.016) (drill 0.508) (layers "F.Cu" "B.Cu") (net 3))
 (via (at 156.1211 132.9436) (size 1.016) (drill 0.508) (layers "F.Cu" "B.Cu") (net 3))
 (via (at 153.5811 122.7836) (size 1.016) (drill 0.508) (layers "F.Cu" "B.Cu") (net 3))
 (segment (start 140.8811 87.2236) (end 140.8811 92.3036) (width 0.4064) (layer "F.Cu") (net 5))
 (segment (start 145.9611 86.8036) (end 141.3011 86.8036) (width 0.4064) (layer "F.Cu") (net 5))
 (segment (start 141.3011 86.8036) (end 140.8811 87.2236) (width 0.4064) (layer "F.Cu") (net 5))
 (via (at 140.8811 122.7836) (size 1.016) (drill 0.508) (layers "F.Cu" "B.Cu") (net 5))
 (via (at 139.6111 107.5436) (size 1.016) (drill 0.508) (layers "F.Cu" "B.Cu") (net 5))
 (via (at 138.3411 112.6236) (size 1.016) (drill 0.508) (layers "F.Cu" "B.Cu") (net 5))
 (via (at 140.8811 92.3036) (size 1.016) (drill 0.508) (layers "F.Cu" "B.Cu") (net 5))
 (via (at 138.3411 92.3036) (size 1.016) (drill 0.508) (layers "F.Cu" "B.Cu") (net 5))
 (via (at 140.8811 102.4636) (size 1.016) (drill 0.508) (layers "F.Cu" "B.Cu") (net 5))
 (via (at 142.1511 127.8636) (size 1.016) (drill 0.508) (layers "F.Cu" "B.Cu") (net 5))
 (via (at 139.6111 117.7036) (size 1.016) (drill 0.508) (layers "F.Cu" "B.Cu") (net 5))
 (via (at 138.3411 122.7836) (size 1.016) (drill 0.508) (layers "F.Cu" "B.Cu") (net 5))
 (via (at 142.1511 117.7036) (size 1.016) (drill 0.508) (layers "F.Cu" "B.Cu") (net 5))
 (via (at 139.6111 127.8636) (size 1.016) (drill 0.508) (layers "F.Cu" "B.Cu") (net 5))
 (via (at 143.4211 92.3036) (size 1.016) (drill 0.508) (layers "F.Cu" "B.Cu") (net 5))
 (via (at 139.6111 97.3836) (size 1.016) (drill 0.508) (layers "F.Cu" "B.Cu") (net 5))
 (via (at 138.3411 102.4636) (size 1.016) (drill 0.508) (layers "F.Cu" "B.Cu") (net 5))
 (via (at 143.4211 122.7836) (size 1.016) (drill 0.508) (layers "F.Cu" "B.Cu") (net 5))
 (via (at 142.1511 97.3836) (size 1.016) (drill 0.508) (layers "F.Cu" "B.Cu") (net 5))
 (via (at 140.8811 132.9436) (size 1.016) (drill 0.508) (layers "F.Cu" "B.Cu") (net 5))
 (via (at 140.8811 112.6236) (size 1.016) (drill 0.508) (layers "F.Cu" "B.Cu") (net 5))
 (via (at 143.4211 102.4636) (size 1.016) (drill 0.508) (layers "F.Cu" "B.Cu") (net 5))
 (via (at 143.4211 112.6236) (size 1.016) (drill 0.508) (layers "F.Cu" "B.Cu") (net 5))
 (via (at 142.1511 107.5436) (size 1.016) (drill 0.508) (layers "F.Cu" "B.Cu") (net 5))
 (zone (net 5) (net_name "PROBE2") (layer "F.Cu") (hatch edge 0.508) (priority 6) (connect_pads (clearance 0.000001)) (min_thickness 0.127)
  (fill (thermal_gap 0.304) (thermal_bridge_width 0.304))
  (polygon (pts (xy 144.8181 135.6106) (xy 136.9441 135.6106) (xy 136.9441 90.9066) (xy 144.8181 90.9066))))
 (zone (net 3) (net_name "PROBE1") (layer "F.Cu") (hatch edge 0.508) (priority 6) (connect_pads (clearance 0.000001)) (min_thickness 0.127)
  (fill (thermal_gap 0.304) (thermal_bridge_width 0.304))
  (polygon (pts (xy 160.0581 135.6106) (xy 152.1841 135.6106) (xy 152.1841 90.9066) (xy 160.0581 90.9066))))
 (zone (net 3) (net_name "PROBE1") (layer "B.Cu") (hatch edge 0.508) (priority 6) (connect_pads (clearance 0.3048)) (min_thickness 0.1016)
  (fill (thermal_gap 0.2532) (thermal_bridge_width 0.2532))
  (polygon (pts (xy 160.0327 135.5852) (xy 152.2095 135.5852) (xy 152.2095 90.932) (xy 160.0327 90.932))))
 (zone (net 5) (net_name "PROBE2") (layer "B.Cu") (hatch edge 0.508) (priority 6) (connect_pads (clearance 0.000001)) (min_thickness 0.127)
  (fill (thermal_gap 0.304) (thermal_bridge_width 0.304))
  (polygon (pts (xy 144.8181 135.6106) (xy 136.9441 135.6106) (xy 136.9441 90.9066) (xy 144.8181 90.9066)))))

